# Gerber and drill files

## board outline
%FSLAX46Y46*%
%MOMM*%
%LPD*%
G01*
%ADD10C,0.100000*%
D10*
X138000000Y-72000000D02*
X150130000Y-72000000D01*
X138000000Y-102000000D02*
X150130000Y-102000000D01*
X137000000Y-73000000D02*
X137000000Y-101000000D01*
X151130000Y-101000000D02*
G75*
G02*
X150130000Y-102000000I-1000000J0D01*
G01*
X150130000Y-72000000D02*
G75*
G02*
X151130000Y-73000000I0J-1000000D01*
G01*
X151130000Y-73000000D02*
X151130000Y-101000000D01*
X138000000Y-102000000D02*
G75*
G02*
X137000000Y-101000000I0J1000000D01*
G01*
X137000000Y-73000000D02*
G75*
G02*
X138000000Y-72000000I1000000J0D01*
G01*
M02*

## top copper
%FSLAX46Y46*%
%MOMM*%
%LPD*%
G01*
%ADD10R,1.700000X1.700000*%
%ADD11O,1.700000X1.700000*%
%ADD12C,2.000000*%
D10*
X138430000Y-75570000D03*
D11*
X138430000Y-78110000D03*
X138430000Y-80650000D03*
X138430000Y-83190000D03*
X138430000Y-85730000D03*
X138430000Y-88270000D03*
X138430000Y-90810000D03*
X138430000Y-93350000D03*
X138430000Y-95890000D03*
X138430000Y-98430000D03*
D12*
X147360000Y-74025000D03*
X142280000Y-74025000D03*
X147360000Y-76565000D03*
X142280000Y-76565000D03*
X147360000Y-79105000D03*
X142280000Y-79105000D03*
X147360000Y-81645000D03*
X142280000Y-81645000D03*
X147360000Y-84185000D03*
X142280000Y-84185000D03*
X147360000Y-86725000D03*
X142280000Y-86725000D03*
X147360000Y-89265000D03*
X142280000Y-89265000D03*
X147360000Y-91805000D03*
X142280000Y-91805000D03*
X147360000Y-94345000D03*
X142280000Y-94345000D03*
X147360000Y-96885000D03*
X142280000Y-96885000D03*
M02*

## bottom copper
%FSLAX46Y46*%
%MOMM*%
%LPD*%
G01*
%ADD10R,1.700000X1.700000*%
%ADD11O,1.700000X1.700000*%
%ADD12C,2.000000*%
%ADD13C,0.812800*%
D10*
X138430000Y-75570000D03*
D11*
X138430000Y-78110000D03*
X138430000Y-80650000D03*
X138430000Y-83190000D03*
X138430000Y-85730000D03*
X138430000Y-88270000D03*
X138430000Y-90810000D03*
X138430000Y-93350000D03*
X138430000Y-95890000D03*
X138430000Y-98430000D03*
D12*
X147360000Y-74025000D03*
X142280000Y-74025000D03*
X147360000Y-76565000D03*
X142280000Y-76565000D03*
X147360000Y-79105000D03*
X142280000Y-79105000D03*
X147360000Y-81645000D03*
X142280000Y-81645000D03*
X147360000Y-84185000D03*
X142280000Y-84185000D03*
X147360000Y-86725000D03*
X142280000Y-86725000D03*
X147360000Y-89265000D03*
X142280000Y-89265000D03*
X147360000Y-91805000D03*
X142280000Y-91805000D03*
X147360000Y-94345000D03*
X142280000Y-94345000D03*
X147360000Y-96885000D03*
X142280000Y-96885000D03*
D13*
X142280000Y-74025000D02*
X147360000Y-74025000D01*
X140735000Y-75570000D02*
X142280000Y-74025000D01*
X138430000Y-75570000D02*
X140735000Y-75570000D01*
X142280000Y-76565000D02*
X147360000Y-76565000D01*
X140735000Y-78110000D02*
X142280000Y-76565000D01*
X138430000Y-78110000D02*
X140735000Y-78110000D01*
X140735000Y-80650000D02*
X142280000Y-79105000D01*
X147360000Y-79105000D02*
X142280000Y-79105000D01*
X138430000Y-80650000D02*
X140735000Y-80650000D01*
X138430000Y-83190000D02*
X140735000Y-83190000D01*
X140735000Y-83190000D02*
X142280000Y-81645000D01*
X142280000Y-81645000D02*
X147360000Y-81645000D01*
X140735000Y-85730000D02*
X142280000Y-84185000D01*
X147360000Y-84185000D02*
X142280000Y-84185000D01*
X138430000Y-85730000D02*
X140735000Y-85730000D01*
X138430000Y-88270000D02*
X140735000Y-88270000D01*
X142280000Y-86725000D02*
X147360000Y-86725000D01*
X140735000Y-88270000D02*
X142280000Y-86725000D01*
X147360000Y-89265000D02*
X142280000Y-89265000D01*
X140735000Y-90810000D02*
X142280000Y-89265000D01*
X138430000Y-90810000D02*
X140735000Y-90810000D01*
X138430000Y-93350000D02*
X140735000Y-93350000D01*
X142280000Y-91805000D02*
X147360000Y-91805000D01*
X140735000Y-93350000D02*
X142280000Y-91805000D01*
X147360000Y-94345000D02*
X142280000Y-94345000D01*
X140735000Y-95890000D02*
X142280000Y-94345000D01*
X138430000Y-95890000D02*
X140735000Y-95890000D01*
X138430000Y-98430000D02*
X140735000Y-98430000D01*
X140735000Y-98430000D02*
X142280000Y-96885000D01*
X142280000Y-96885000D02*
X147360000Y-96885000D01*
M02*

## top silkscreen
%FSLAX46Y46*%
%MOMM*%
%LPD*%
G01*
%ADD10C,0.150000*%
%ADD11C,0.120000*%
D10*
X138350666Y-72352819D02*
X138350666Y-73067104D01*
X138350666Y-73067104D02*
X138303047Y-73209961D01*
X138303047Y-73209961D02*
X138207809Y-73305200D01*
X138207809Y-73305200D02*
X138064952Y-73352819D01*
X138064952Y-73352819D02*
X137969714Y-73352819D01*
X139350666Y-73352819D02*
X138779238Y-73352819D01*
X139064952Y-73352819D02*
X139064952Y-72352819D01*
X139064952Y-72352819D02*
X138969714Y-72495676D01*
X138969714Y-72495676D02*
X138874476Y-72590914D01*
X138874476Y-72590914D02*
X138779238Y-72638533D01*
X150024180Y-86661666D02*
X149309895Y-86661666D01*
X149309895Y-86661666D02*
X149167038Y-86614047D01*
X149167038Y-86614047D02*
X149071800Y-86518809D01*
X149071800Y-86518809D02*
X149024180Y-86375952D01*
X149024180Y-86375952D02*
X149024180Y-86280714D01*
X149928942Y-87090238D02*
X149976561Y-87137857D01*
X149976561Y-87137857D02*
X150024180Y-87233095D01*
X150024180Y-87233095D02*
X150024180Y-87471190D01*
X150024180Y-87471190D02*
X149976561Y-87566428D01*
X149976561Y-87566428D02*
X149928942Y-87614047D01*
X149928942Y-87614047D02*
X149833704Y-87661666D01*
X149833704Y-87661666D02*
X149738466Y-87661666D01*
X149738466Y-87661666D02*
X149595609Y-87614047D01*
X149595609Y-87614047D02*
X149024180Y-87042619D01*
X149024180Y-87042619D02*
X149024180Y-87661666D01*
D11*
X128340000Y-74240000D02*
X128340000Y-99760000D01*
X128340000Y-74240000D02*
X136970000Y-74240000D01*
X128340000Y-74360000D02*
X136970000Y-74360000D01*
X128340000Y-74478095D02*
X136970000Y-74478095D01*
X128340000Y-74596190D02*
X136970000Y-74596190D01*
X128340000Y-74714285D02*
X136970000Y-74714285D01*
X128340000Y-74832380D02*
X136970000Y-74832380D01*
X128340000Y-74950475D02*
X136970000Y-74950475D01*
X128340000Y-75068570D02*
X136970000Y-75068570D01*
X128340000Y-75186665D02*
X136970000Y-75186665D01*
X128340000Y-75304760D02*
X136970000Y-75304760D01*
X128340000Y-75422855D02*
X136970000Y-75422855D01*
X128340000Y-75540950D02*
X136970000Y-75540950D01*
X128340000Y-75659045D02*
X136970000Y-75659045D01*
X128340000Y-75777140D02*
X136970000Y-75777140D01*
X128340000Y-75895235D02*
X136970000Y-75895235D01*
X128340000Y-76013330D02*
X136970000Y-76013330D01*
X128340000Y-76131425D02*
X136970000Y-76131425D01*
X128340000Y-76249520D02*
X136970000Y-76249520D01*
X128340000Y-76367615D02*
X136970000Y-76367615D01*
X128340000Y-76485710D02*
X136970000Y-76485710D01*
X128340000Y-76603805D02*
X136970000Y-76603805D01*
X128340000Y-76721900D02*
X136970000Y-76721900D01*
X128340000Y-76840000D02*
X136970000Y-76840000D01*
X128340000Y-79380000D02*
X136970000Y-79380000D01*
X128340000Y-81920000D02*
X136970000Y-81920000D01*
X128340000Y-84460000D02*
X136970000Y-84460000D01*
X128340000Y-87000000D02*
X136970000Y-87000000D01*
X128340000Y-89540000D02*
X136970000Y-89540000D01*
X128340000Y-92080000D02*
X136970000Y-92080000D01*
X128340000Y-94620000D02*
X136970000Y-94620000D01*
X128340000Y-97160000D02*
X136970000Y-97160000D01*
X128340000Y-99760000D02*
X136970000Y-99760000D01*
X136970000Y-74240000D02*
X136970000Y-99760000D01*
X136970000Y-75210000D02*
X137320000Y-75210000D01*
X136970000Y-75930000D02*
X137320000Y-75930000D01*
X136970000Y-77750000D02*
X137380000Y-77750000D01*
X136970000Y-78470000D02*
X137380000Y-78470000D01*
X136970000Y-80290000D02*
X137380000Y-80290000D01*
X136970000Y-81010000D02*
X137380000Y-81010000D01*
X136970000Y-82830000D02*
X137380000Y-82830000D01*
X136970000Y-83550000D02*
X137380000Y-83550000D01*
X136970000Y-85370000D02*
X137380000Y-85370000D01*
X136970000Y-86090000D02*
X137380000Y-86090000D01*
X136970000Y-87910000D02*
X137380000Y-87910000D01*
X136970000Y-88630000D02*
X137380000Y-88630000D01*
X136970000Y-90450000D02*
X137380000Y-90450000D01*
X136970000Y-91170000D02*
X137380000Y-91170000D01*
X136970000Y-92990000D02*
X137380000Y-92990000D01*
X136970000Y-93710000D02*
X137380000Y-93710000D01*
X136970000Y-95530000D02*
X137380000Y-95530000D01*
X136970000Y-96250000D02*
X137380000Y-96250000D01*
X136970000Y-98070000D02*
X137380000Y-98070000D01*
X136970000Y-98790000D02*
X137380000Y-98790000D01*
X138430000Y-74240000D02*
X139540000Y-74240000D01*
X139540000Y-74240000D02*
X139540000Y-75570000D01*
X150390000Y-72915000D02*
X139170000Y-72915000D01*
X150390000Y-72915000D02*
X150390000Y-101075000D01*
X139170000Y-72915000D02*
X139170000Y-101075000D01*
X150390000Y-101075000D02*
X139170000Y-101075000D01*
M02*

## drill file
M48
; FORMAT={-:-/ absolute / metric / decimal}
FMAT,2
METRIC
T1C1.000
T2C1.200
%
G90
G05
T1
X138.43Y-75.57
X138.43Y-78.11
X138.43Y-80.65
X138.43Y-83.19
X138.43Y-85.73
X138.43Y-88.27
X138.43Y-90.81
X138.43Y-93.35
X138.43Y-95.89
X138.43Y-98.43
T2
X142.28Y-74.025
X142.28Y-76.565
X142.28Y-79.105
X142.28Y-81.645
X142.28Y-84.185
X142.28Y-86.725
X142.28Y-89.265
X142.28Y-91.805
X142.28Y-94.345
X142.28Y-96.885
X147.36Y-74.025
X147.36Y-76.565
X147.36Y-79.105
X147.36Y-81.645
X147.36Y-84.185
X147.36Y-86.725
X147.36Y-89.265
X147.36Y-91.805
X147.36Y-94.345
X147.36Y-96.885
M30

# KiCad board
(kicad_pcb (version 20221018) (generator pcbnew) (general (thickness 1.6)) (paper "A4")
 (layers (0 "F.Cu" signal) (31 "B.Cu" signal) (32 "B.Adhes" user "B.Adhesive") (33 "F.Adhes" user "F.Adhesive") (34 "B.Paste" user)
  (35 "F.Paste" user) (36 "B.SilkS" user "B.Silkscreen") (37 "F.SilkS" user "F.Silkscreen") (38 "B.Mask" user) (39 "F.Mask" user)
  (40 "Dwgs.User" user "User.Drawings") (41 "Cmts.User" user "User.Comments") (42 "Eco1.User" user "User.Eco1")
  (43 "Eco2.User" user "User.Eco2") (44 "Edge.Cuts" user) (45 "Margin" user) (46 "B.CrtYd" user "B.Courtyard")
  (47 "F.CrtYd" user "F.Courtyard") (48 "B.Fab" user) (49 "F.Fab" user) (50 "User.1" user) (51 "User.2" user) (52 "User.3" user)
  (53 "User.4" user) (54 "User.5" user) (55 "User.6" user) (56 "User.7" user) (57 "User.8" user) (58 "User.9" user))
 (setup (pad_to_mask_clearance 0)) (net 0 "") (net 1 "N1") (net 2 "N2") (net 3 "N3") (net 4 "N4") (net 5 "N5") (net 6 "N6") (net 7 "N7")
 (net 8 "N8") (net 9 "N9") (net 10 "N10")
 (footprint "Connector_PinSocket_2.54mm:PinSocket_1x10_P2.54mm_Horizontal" (layer "F.Cu") (at 138.43 75.57)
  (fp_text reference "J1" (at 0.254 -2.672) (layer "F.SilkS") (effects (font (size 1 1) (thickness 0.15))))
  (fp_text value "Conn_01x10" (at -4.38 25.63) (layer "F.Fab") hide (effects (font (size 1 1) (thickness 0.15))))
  (fp_line (start -10.09 -1.33) (end -10.09 24.19) (stroke (width 0.12) (type solid)) (layer "F.SilkS"))
  (fp_line (start -10.09 -1.33) (end -1.46 -1.33) (stroke (width 0.12) (type solid)) (layer "F.SilkS"))
  (fp_line (start -10.09 -1.21) (end -1.46 -1.21) (stroke (width 0.12) (type solid)) (layer "F.SilkS"))
  (fp_line (start -10.09 -1.091905) (end -1.46 -1.091905) (stroke (width 0.12) (type solid)) (layer "F.SilkS"))
  (fp_line (start -10.09 -0.97381) (end -1.46 -0.97381) (stroke (width 0.12) (type solid)) (layer "F.SilkS"))
  (fp_line (start -10.09 -0.855715) (end -1.46 -0.855715) (stroke (width 0.12) (type solid)) (layer "F.SilkS"))
  (fp_line (start -10.09 -0.73762) (end -1.46 -0.73762) (stroke (width 0.12) (type solid)) (layer "F.SilkS"))
  (fp_line (start -10.09 -0.619525) (end -1.46 -0.619525) (stroke (width 0.12) (type solid)) (layer "F.SilkS"))
  (fp_line (start -10.09 -0.50143) (end -1.46 -0.50143) (stroke (width 0.12) (type solid)) (layer "F.SilkS"))
  (fp_line (start -10.09 -0.383335) (end -1.46 -0.383335) (stroke (width 0.12) (type solid)) (layer "F.SilkS"))
  (fp_line (start -10.09 -0.26524) (end -1.46 -0.26524) (stroke (width 0.12) (type solid)) (layer "F.SilkS"))
  (fp_line (start -10.09 -0.147145) (end -1.46 -0.147145) (stroke (width 0.12) (type solid)) (layer "F.SilkS"))
  (fp_line (start -10.09 -0.02905) (end -1.46 -0.02905) (stroke (width 0.12) (type solid)) (layer "F.SilkS"))
  (fp_line (start -10.09 0.089045) (end -1.46 0.089045) (stroke (width 0.12) (type solid)) (layer "F.SilkS"))
  (fp_line (start -10.09 0.20714) (end -1.46 0.20714) (stroke (width 0.12) (type solid)) (layer "F.SilkS"))
  (fp_line (start -10.09 0.325235) (end -1.46 0.325235) (stroke (width 0.12) (type solid)) (layer "F.SilkS"))
  (fp_line (start -10.09 0.44333) (end -1.46 0.44333) (stroke (width 0.12) (type solid)) (layer "F.SilkS"))
  (fp_line (start -10.09 0.561425) (end -1.46 0.561425) (stroke (width 0.12) (type solid)) (layer "F.SilkS"))
  (fp_line (start -10.09 0.67952) (end -1.46 0.67952) (stroke (width 0.12) (type solid)) (layer "F.SilkS"))
  (fp_line (start -10.09 0.797615) (end -1.46 0.797615) (stroke (width 0.12) (type solid)) (layer "F.SilkS"))
  (fp_line (start -10.09 0.91571) (end -1.46 0.91571) (stroke (width 0.12) (type solid)) (layer "F.SilkS"))
  (fp_line (start -10.09 1.033805) (end -1.46 1.033805) (stroke (width 0.12) (type solid)) (layer "F.SilkS"))
  (fp_line (start -10.09 1.1519) (end -1.46 1.1519) (stroke (width 0.12) (type solid)) (layer "F.SilkS"))
  (fp_line (start -10.09 1.27) (end -1.46 1.27) (stroke (width 0.12) (type solid)) (layer "F.SilkS"))
  (fp_line (start -10.09 3.81) (end -1.46 3.81) (stroke (width 0.12) (type solid)) (layer "F.SilkS"))
  (fp_line (start -10.09 6.35) (end -1.46 6.35) (stroke (width 0.12) (type solid)) (layer "F.SilkS"))
  (fp_line (start -10.09 8.89) (end -1.46 8.89) (stroke (width 0.12) (type solid)) (layer "F.SilkS"))
  (fp_line (start -10.09 11.43) (end -1.46 11.43) (stroke (width 0.12) (type solid)) (layer "F.SilkS"))
  (fp_line (start -10.09 13.97) (end -1.46 13.97) (stroke (width 0.12) (type solid)) (layer "F.SilkS"))
  (fp_line (start -10.09 16.51) (end -1.46 16.51) (stroke (width 0.12) (type solid)) (layer "F.SilkS"))
  (fp_line (start -10.09 19.05) (end -1.46 19.05) (stroke (width 0.12) (type solid)) (layer "F.SilkS"))
  (fp_line (start -10.09 21.59) (end -1.46 21.59) (stroke (width 0.12) (type solid)) (layer "F.SilkS"))
  (fp_line (start -10.09 24.19) (end -1.46 24.19) (stroke (width 0.12) (type solid)) (layer "F.SilkS"))
  (fp_line (start -1.46 -1.33) (end -1.46 24.19) (stroke (width 0.12) (type solid)) (layer "F.SilkS"))
  (fp_line (start -1.46 -0.36) (end -1.11 -0.36) (stroke (width 0.12) (type solid)) (layer "F.SilkS"))
  (fp_line (start -1.46 0.36) (end -1.11 0.36) (stroke (width 0.12) (type solid)) (layer "F.SilkS"))
  (fp_line (start -1.46 2.18) (end -1.05 2.18) (stroke (width 0.12) (type solid)) (layer "F.SilkS"))
  (fp_line (start -1.46 2.9) (end -1.05 2.9) (stroke (width 0.12) (type solid)) (layer "F.SilkS"))
  (fp_line (start -1.46 4.72) (end -1.05 4.72) (stroke (width 0.12) (type solid)) (layer "F.SilkS"))
  (fp_line (start -1.46 5.44) (end -1.05 5.44) (stroke (width 0.12) (type solid)) (layer "F.SilkS"))
  (fp_line (start -1.46 7.26) (end -1.05 7.26) (stroke (width 0.12) (type solid)) (layer "F.SilkS"))
  (fp_line (start -1.46 7.98) (end -1.05 7.98) (stroke (width 0.12) (type solid)) (layer "F.SilkS"))
  (fp_line (start -1.46 9.8) (end -1.05 9.8) (stroke (width 0.12) (type solid)) (layer "F.SilkS"))
  (fp_line (start -1.46 10.52) (end -1.05 10.52) (stroke (width 0.12) (type solid)) (layer "F.SilkS"))
  (fp_line (start -1.46 12.34) (end -1.05 12.34) (stroke (width 0.12) (type solid)) (layer "F.SilkS"))
  (fp_line (start -1.46 13.06) (end -1.05 13.06) (stroke (width 0.12) (type solid)) (layer "F.SilkS"))
  (fp_line (start -1.46 14.88) (end -1.05 14.88) (stroke (width 0.12) (type solid)) (layer "F.SilkS"))
  (fp_line (start -1.46 15.6) (end -1.05 15.6) (stroke (width 0.12) (type solid)) (layer "F.SilkS"))
  (fp_line (start -1.46 17.42) (end -1.05 17.42) (stroke (width 0.12) (type solid)) (layer "F.SilkS"))
  (fp_line (start -1.46 18.14) (end -1.05 18.14) (stroke (width 0.12) (type solid)) (layer "F.SilkS"))
  (fp_line (start -1.46 19.96) (end -1.05 19.96) (stroke (width 0.12) (type solid)) (layer "F.SilkS"))
  (fp_line (start -1.46 20.68) (end -1.05 20.68) (stroke (width 0.12) (type solid)) (layer "F.SilkS"))
  (fp_line (start -1.46 22.5) (end -1.05 22.5) (stroke (width 0.12) (type solid)) (layer "F.SilkS"))
  (fp_line (start -1.46 23.22) (end -1.05 23.22) (stroke (width 0.12) (type solid)) (layer "F.SilkS"))
  (fp_line (start 0 -1.33) (end 1.11 -1.33) (stroke (width 0.12) (type solid)) (layer "F.SilkS"))
  (fp_line (start 1.11 -1.33) (end 1.11 0) (stroke (width 0.12) (type solid)) (layer "F.SilkS"))
  (pad "1" thru_hole rect (at 0 0) (size 1.7 1.7) (drill 1) (layers "*.Cu" "*.Mask") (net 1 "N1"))
  (pad "2" thru_hole oval (at 0 2.54) (size 1.7 1.7) (drill 1) (layers "*.Cu" "*.Mask") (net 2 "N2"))
  (pad "3" thru_hole oval (at 0 5.08) (size 1.7 1.7) (drill 1) (layers "*.Cu" "*.Mask") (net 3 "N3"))
  (pad "4" thru_hole oval (at 0 7.62) (size 1.7 1.7) (drill 1) (layers "*.Cu" "*.Mask") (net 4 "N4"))
  (pad "5" thru_hole oval (at 0 10.16) (size 1.7 1.7) (drill 1) (layers "*.Cu" "*.Mask") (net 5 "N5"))
  (pad "6" thru_hole oval (at 0 12.7) (size 1.7 1.7) (drill 1) (layers "*.Cu" "*.Mask") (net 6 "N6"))
  (pad "7" thru_hole oval (at 0 15.24) (size 1.7 1.7) (drill 1) (layers "*.Cu" "*.Mask") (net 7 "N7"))
  (pad "8" thru_hole oval (at 0 17.78) (size 1.7 1.7) (drill 1) (layers "*.Cu" "*.Mask") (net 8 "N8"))
  (pad "9" thru_hole oval (at 0 20.32) (size 1.7 1.7) (drill 1) (layers "*.Cu" "*.Mask") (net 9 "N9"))
  (pad "10" thru_hole oval (at 0 22.86) (size 1.7 1.7) (drill 1) (layers "*.Cu" "*.Mask") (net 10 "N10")))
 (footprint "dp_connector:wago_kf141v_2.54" (layer "F.Cu") (at 144.78 86.995 -90)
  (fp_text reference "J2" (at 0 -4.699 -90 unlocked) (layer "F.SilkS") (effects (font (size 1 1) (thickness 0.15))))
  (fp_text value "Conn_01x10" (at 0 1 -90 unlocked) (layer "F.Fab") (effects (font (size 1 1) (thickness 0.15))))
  (fp_line (start -14.08 -5.61) (end -14.08 5.61) (stroke (width 0.12) (type default)) (layer "F.SilkS"))
  (fp_line (start -14.08 -5.61) (end 14.08 -5.61) (stroke (width 0.12) (type default)) (layer "F.SilkS"))
  (fp_line (start -14.08 5.61) (end 14.08 5.61) (stroke (width 0.12) (type default)) (layer "F.SilkS"))
  (fp_line (start 14.08 -5.61) (end 14.08 5.61) (stroke (width 0.12) (type default)) (layer "F.SilkS"))
  (pad "1" thru_hole circle (at -12.97 -2.58 270) (size 2 2) (drill 1.2) (layers "*.Cu" "*.Mask") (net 1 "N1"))
  (pad "1" thru_hole circle (at -12.97 2.5 270) (size 2 2) (drill 1.2) (layers "*.Cu" "*.Mask") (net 1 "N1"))
  (pad "2" thru_hole circle (at -10.43 -2.58 270) (size 2 2) (drill 1.2) (layers "*.Cu" "*.Mask") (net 2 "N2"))
  (pad "2" thru_hole circle (at -10.43 2.5 270) (size 2 2) (drill 1.2) (layers "*.Cu" "*.Mask") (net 2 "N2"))
  (pad "3" thru_hole circle (at -7.89 -2.58 270) (size 2 2) (drill 1.2) (layers "*.Cu" "*.Mask") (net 3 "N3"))
  (pad "3" thru_hole circle (at -7.89 2.5 270) (size 2 2) (drill 1.2) (layers "*.Cu" "*.Mask") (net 3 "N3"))
  (pad "4" thru_hole circle (at -5.35 -2.58 270) (size 2 2) (drill 1.2) (layers "*.Cu" "*.Mask") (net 4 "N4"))
  (pad "4" thru_hole circle (at -5.35 2.5 270) (size 2 2) (drill 1.2) (layers "*.Cu" "*.Mask") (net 4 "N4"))
  (pad "5" thru_hole circle (at -2.81 -2.58 270) (size 2 2) (drill 1.2) (layers "*.Cu" "*.Mask") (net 5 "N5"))
  (pad "5" thru_hole circle (at -2.81 2.5 270) (size 2 2) (drill 1.2) (layers "*.Cu" "*.Mask") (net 5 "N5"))
  (pad "6" thru_hole circle (at -0.27 -2.58 270) (size 2 2) (drill 1.2) (layers "*.Cu" "*.Mask") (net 6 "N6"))
  (pad "6" thru_hole circle (at -0.27 2.5 270) (size 2 2) (drill 1.2) (layers "*.Cu" "*.Mask") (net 6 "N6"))
  (pad "7" thru_hole circle (at 2.27 -2.58 270) (size 2 2) (drill 1.2) (layers "*.Cu" "*.Mask") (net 7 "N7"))
  (pad "7" thru_hole circle (at 2.27 2.5 270) (size 2 2) (drill 1.2) (layers "*.Cu" "*.Mask") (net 7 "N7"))
  (pad "8" thru_hole circle (at 4.81 -2.58 270) (size 2 2) (drill 1.2) (layers "*.Cu" "*.Mask") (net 8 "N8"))
  (pad "8" thru_hole circle (at 4.81 2.5 270) (size 2 2) (drill 1.2) (layers "*.Cu" "*.Mask") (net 8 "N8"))
  (pad "9" thru_hole circle (at 7.35 -2.58 270) (size 2 2) (drill 1.2) (layers "*.Cu" "*.Mask") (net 9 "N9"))
  (pad "9" thru_hole circle (at 7.35 2.5 270) (size 2 2) (drill 1.2) (layers "*.Cu" "*.Mask") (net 9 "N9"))
  (pad "10" thru_hole circle (at 9.89 -2.58 270) (size 2 2) (drill 1.2) (layers "*.Cu" "*.Mask") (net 10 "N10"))
  (pad "10" thru_hole circle (at 9.89 2.5 270) (size 2 2) (drill 1.2) (layers "*.Cu" "*.Mask") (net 10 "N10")))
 (gr_line (start 138 72) (end 150.13 72) (stroke (width 0.1) (type default)) (layer "Edge.Cuts"))
 (gr_line (start 138 102) (end 150.13 102) (stroke (width 0.1) (type default)) (layer "Edge.Cuts"))
 (gr_line (start 137 73) (end 137 101) (stroke (width 0.1) (type default)) (layer "Edge.Cuts"))
 (gr_arc (start 151.13 101) (mid 150.837107 101.707107) (end 150.13 102) (stroke (width 0.1) (type default)) (layer "Edge.Cuts"))
 (gr_arc (start 150.13 72) (mid 150.837107 72.292893) (end 151.13 73) (stroke (width 0.1) (type default)) (layer "Edge.Cuts"))
 (gr_line (start 151.13 73) (end 151.13 101) (stroke (width 0.1) (type default)) (layer "Edge.Cuts"))
 (gr_arc (start 138 102) (mid 137.292893 101.707107) (end 137 101) (stroke (width 0.1) (type default)) (layer "Edge.Cuts"))
 (gr_arc (start 137 73) (mid 137.292893 72.292893) (end 138 72) (stroke (width 0.1) (type default)) (layer "Edge.Cuts"))
 (segment (start 142.28 74.025) (end 147.36 74.025) (width 0.8128) (layer "B.Cu") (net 1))
 (segment (start 140.735 75.57) (end 142.28 74.025) (width 0.8128) (layer "B.Cu") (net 1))
 (segment (start 138.43 75.57) (end 140.735 75.57) (width 0.8128) (layer "B.Cu") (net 1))
 (segment (start 142.28 76.565) (end 147.36 76.565) (width 0.8128) (layer "B.Cu") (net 2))
 (segment (start 140.735 78.11) (end 142.28 76.565) (width 0.8128) (layer "B.Cu") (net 2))
 (segment (start 138.43 78.11) (end 140.735 78.11) (width 0.8128) (layer "B.Cu") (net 2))
 (segment (start 140.735 80.65) (end 142.28 79.105) (width 0.8128) (layer "B.Cu") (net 3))
 (segment (start 147.36 79.105) (end 142.28 79.105) (width 0.8128) (layer "B.Cu") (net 3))
 (segment (start 138.43 80.65) (end 140.735 80.65) (width 0.8128) (layer "B.Cu") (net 3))
 (segment (start 138.43 83.19) (end 140.735 83.19) (width 0.8128) (layer "B.Cu") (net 4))
 (segment (start 140.735 83.19) (end 142.28 81.645) (width 0.8128) (layer "B.Cu") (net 4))
 (segment (start 142.28 81.645) (end 147.36 81.645) (width 0.8128) (layer "B.Cu") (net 4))
 (segment (start 140.735 85.73) (end 142.28 84.185) (width 0.8128) (layer "B.Cu") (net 5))
 (segment (start 147.36 84.185) (end 142.28 84.185) (width 0.8128) (layer "B.Cu") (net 5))
 (segment (start 138.43 85.73) (end 140.735 85.73) (width 0.8128) (layer "B.Cu") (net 5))
 (segment (start 138.43 88.27) (end 140.735 88.27) (width 0.8128) (layer "B.Cu") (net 6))
 (segment (start 142.28 86.725) (end 147.36 86.725) (width 0.8128) (layer "B.Cu") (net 6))
 (segment (start 140.735 88.27) (end 142.28 86.725) (width 0.8128) (layer "B.Cu") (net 6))
 (segment (start 147.36 89.265) (end 142.28 89.265) (width 0.8128) (layer "B.Cu") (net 7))
 (segment (start 140.735 90.81) (end 142.28 89.265) (width 0.8128) (layer "B.Cu") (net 7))
 (segment (start 138.43 90.81) (end 140.735 90.81) (width 0.8128) (layer "B.Cu") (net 7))
 (segment (start 138.43 93.35) (end 140.735 93.35) (width 0.8128) (layer "B.Cu") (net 8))
 (segment (start 142.28 91.805) (end 147.36 91.805) (width 0.8128) (layer "B.Cu") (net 8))
 (segment (start 140.735 93.35) (end 142.28 91.805) (width 0.8128) (layer "B.Cu") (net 8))
 (segment (start 147.36 94.345) (end 142.28 94.345) (width 0.8128) (layer "B.Cu") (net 9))
 (segment (start 140.735 95.89) (end 142.28 94.345) (width 0.8128) (layer "B.Cu") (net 9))
 (segment (start 138.43 95.89) (end 140.735 95.89) (width 0.8128) (layer "B.Cu") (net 9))
 (segment (start 138.43 98.43) (end 140.735 98.43) (width 0.8128) (layer "B.Cu") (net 10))
 (segment (start 140.735 98.43) (end 142.28 96.885) (width 0.8128) (layer "B.Cu") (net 10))
 (segment (start 142.28 96.885) (end 147.36 96.885) (width 0.8128) (layer "B.Cu") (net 10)))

